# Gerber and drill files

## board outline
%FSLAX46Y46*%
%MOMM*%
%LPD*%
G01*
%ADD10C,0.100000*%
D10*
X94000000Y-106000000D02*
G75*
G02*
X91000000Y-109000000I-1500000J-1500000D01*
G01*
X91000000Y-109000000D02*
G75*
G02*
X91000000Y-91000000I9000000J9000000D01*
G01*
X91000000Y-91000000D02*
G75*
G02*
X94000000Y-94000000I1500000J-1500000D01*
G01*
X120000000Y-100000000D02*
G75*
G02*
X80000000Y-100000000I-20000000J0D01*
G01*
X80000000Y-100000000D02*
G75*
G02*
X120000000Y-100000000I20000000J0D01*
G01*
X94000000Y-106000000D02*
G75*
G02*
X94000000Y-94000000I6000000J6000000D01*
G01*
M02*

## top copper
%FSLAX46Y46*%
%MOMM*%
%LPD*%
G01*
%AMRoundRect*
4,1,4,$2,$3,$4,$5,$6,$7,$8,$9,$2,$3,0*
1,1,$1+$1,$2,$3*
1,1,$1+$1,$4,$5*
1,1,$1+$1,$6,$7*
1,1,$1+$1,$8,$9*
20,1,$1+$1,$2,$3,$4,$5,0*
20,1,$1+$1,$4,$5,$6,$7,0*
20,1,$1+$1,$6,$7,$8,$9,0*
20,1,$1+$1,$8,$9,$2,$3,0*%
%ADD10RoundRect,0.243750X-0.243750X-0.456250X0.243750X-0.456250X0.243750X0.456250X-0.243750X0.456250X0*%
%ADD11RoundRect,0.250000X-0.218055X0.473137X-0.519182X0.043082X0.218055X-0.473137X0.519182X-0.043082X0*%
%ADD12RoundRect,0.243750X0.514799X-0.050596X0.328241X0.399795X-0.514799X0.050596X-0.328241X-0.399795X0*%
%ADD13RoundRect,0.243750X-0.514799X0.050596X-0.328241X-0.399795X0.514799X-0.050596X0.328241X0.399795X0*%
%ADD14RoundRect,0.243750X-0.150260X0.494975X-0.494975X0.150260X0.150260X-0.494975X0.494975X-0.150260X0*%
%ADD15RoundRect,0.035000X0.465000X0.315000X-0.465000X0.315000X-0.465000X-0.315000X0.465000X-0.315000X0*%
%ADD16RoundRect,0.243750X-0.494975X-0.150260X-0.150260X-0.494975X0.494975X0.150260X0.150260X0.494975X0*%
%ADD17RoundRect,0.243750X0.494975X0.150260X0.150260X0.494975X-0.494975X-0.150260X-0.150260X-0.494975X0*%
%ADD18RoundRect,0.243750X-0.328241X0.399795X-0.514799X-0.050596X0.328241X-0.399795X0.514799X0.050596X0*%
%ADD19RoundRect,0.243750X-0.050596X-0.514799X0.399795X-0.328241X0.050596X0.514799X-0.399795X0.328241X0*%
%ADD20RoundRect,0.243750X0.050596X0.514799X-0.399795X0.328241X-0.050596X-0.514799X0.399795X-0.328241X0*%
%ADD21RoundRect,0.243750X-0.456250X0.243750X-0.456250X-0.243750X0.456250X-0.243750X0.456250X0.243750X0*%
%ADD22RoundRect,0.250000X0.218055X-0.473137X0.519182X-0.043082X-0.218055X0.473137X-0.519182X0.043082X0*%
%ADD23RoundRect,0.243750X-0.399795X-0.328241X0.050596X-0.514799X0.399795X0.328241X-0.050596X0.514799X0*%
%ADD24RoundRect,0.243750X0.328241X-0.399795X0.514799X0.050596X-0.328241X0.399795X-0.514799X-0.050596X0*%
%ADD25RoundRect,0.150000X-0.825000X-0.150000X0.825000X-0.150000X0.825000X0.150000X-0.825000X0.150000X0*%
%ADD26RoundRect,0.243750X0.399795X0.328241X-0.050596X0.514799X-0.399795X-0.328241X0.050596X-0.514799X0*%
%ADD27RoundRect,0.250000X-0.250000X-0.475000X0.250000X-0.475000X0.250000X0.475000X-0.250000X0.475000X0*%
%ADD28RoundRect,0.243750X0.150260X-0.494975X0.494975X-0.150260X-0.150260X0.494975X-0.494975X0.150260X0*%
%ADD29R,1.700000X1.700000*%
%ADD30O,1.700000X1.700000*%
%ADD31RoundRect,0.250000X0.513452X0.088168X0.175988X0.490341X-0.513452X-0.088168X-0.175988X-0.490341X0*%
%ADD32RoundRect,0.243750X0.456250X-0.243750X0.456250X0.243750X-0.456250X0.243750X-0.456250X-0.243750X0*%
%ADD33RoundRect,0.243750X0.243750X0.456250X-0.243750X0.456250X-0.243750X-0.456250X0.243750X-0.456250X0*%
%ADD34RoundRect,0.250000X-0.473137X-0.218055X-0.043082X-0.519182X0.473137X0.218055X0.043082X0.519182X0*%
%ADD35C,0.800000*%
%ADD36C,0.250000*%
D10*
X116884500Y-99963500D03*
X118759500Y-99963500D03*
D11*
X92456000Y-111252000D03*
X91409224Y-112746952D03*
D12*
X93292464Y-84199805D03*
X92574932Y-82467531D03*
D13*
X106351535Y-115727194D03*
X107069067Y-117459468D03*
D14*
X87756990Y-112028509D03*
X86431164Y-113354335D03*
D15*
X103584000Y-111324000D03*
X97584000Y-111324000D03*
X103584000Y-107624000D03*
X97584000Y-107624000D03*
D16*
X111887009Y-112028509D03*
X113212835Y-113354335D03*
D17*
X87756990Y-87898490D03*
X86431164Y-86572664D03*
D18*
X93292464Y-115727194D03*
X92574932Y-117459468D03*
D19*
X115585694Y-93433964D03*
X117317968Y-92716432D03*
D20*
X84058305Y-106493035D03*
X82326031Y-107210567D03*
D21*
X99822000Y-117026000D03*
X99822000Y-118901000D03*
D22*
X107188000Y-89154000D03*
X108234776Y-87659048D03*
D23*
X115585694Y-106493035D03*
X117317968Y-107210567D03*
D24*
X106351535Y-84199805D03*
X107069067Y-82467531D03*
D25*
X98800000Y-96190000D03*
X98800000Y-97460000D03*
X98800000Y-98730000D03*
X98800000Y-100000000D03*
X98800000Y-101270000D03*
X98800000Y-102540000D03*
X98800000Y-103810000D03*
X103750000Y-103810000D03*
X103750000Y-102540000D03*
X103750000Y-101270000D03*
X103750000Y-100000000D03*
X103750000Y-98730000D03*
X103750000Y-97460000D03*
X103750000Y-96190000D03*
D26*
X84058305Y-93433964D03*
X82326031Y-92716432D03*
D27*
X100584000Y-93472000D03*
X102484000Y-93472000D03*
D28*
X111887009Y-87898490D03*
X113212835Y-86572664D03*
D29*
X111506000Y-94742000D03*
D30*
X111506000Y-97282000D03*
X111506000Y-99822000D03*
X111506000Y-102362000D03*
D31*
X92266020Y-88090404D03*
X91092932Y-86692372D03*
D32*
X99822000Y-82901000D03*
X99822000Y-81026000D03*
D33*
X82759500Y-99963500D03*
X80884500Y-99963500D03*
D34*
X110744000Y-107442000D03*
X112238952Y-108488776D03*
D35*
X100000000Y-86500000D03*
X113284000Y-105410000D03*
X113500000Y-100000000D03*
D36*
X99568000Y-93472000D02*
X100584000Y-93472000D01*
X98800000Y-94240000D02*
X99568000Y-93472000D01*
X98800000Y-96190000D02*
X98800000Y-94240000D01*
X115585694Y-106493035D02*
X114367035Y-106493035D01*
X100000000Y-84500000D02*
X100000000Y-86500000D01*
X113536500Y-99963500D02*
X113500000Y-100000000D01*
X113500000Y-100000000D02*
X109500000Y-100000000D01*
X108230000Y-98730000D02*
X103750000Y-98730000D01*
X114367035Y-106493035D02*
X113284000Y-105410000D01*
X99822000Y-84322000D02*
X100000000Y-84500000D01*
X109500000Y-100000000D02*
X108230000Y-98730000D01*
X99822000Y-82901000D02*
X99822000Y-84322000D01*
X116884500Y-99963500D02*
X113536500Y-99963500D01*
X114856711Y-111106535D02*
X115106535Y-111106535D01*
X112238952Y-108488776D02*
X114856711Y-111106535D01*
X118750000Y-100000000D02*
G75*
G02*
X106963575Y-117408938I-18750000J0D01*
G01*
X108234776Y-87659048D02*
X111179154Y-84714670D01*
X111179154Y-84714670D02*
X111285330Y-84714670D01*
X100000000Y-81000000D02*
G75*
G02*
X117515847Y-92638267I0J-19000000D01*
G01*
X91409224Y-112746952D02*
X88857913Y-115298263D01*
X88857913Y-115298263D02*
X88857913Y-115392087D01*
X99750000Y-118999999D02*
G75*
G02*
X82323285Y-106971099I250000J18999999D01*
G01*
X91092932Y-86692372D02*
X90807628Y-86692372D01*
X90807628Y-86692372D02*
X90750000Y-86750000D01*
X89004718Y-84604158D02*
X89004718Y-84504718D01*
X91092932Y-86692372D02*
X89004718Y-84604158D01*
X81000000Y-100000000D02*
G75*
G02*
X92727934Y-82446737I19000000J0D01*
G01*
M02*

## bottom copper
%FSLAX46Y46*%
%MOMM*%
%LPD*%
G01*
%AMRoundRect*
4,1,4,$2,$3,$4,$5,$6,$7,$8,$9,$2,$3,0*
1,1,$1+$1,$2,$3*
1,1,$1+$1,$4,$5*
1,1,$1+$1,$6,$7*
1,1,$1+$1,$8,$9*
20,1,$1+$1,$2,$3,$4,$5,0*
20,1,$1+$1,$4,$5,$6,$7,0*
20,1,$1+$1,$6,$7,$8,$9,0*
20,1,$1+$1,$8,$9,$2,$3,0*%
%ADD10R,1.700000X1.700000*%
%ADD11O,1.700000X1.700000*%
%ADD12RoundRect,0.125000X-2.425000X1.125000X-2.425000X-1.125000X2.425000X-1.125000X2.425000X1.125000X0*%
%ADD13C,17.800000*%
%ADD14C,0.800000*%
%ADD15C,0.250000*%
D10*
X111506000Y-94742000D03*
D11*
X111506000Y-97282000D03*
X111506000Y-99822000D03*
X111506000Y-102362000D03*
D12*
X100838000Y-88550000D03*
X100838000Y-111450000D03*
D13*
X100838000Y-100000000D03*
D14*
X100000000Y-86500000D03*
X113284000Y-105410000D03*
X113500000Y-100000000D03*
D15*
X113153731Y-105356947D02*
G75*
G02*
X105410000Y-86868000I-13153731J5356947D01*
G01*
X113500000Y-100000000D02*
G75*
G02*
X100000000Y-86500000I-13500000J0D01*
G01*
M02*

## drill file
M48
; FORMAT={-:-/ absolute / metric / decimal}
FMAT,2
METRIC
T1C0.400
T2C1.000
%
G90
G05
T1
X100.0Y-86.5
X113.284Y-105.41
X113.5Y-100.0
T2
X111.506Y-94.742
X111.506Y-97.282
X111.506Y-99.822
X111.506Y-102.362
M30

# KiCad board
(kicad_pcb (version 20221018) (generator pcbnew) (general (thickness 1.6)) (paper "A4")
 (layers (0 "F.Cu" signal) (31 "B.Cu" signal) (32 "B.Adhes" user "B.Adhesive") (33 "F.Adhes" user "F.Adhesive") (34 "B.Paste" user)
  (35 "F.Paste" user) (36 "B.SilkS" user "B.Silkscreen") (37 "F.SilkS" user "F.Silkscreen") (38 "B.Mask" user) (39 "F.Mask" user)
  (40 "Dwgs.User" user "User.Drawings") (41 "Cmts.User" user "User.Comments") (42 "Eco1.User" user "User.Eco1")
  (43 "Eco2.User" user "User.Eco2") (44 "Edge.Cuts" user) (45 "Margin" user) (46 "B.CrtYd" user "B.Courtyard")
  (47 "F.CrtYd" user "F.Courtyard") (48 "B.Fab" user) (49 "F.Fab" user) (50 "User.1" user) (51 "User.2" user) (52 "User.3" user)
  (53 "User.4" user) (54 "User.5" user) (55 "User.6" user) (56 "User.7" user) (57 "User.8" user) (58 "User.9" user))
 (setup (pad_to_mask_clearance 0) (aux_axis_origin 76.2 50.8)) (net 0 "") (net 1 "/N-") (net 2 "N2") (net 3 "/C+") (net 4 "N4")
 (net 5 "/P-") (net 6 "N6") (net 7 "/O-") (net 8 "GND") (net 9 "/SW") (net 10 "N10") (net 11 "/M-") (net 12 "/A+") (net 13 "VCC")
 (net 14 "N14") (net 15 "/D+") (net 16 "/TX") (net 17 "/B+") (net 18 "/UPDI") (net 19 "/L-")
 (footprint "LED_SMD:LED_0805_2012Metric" (layer "F.Cu") (at 117.822 99.9635)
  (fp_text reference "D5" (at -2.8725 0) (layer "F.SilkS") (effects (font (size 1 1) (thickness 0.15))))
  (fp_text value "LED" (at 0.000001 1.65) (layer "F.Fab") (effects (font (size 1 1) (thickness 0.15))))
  (pad "1" smd roundrect (at -0.9375 0) (size 0.975 1.4) (layers "F.Cu" "F.Paste" "F.Mask") (roundrect_rratio 0.25) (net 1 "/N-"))
  (pad "2" smd roundrect (at 0.9375 0) (size 0.975 1.4) (layers "F.Cu" "F.Paste" "F.Mask") (roundrect_rratio 0.25) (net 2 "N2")))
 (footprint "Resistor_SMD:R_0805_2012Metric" (layer "F.Cu") (at 91.932612 111.999476 -125)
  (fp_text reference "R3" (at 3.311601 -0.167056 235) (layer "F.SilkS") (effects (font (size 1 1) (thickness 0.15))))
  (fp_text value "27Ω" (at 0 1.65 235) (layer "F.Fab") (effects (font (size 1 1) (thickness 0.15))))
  (pad "1" smd roundrect (at -0.9125 0 235) (size 1.025 1.4) (layers "F.Cu" "F.Paste" "F.Mask") (roundrect_rratio 0.243902) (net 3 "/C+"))
  (pad "2" smd roundrect (at 0.9125 0 235) (size 1.025 1.4) (layers "F.Cu" "F.Paste" "F.Mask") (roundrect_rratio 0.243902) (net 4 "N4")))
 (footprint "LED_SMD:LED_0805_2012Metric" (layer "F.Cu") (at 92.933698 83.333668 112.5)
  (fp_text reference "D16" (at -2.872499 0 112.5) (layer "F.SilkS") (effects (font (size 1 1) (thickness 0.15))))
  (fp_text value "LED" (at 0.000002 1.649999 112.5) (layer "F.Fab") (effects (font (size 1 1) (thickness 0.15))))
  (pad "1" smd roundrect (at -0.9375 0 112.5) (size 0.975 1.4) (layers "F.Cu" "F.Paste" "F.Mask") (roundrect_rratio 0.25) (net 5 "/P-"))
  (pad "2" smd roundrect (at 0.9375 0 112.5) (size 0.975 1.4) (layers "F.Cu" "F.Paste" "F.Mask") (roundrect_rratio 0.25) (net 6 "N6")))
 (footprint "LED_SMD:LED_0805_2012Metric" (layer "F.Cu") (at 106.710301 116.593331 -67.5)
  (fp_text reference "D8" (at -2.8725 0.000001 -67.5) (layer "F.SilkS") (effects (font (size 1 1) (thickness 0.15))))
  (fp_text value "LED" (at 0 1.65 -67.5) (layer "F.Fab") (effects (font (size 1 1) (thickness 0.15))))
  (pad "1" smd roundrect (at -0.9375 0 292.5) (size 0.975 1.4) (layers "F.Cu" "F.Paste" "F.Mask") (roundrect_rratio 0.25) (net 5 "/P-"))
  (pad "2" smd roundrect (at 0.9375 0 292.5) (size 0.975 1.4) (layers "F.Cu" "F.Paste" "F.Mask") (roundrect_rratio 0.25) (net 2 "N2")))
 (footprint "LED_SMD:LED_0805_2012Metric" (layer "F.Cu") (at 87.094077 112.691422 -135)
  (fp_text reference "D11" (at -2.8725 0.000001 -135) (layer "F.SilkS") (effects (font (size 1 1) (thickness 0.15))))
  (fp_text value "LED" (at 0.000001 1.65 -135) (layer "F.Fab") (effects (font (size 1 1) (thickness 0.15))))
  (pad "1" smd roundrect (at -0.9375 0 225) (size 0.975 1.4) (layers "F.Cu" "F.Paste" "F.Mask") (roundrect_rratio 0.25) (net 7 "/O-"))
  (pad "2" smd roundrect (at 0.9375 0 225) (size 0.975 1.4) (layers "F.Cu" "F.Paste" "F.Mask") (roundrect_rratio 0.25) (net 4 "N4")))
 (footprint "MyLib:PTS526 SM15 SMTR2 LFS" (layer "F.Cu") (at 100.584 109.474 180)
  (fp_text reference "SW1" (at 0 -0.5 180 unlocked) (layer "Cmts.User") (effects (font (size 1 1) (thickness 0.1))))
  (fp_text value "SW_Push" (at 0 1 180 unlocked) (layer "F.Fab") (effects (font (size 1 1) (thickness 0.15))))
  (pad "1" smd roundrect (at -3 -1.85 180) (size 1 0.7) (layers "F.Cu" "F.Paste" "F.Mask") (roundrect_rratio 0.05) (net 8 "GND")
   (thermal_bridge_angle 45))
  (pad "1" smd roundrect (at 3 -1.85 180) (size 1 0.7) (layers "F.Cu" "F.Paste" "F.Mask") (roundrect_rratio 0.05) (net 8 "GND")
   (thermal_bridge_angle 45))
  (pad "2" smd roundrect (at -3 1.85 180) (size 1 0.7) (layers "F.Cu" "F.Paste" "F.Mask") (roundrect_rratio 0.05) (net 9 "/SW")
   (thermal_bridge_angle 45))
  (pad "2" smd roundrect (at 3 1.85 180) (size 1 0.7) (layers "F.Cu" "F.Paste" "F.Mask") (roundrect_rratio 0.05) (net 9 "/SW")
   (thermal_bridge_angle 45)))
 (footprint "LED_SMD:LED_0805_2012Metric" (layer "F.Cu") (at 112.549922 112.691422 -45)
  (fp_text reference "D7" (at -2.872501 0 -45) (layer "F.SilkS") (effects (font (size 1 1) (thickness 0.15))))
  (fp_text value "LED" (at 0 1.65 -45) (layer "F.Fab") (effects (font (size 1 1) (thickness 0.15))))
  (pad "1" smd roundrect (at -0.9375 0 315) (size 0.975 1.4) (layers "F.Cu" "F.Paste" "F.Mask") (roundrect_rratio 0.25) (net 7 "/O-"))
  (pad "2" smd roundrect (at 0.9375 0 315) (size 0.975 1.4) (layers "F.Cu" "F.Paste" "F.Mask") (roundrect_rratio 0.25) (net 2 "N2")))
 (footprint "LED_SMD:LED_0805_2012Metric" (layer "F.Cu") (at 87.094077 87.235577 135)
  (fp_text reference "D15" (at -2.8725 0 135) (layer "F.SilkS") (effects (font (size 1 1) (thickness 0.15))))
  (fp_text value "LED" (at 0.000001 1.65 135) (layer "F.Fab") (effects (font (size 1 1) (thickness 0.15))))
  (pad "1" smd roundrect (at -0.9375 0 135) (size 0.975 1.4) (layers "F.Cu" "F.Paste" "F.Mask") (roundrect_rratio 0.25) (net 7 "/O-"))
  (pad "2" smd roundrect (at 0.9375 0 135) (size 0.975 1.4) (layers "F.Cu" "F.Paste" "F.Mask") (roundrect_rratio 0.25) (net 6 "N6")))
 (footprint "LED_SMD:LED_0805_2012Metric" (layer "F.Cu") (at 92.933698 116.593331 -112.5)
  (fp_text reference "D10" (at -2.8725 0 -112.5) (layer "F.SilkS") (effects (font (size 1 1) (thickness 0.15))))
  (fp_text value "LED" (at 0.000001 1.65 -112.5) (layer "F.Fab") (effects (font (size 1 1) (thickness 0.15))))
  (pad "1" smd roundrect (at -0.9375 0 247.5) (size 0.975 1.4) (layers "F.Cu" "F.Paste" "F.Mask") (roundrect_rratio 0.25) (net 1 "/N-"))
  (pad "2" smd roundrect (at 0.9375 0 247.5) (size 0.975 1.4) (layers "F.Cu" "F.Paste" "F.Mask") (roundrect_rratio 0.25) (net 4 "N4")))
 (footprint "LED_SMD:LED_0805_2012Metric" (layer "F.Cu") (at 116.451831 93.075198 22.5)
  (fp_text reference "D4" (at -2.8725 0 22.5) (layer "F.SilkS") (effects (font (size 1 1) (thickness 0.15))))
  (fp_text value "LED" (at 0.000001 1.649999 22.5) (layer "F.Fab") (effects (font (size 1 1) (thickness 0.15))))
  (pad "1" smd roundrect (at -0.9375 0 22.5) (size 0.975 1.4) (layers "F.Cu" "F.Paste" "F.Mask") (roundrect_rratio 0.25) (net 5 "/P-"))
  (pad "2" smd roundrect (at 0.9375 0 22.5) (size 0.975 1.4) (layers "F.Cu" "F.Paste" "F.Mask") (roundrect_rratio 0.25) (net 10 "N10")))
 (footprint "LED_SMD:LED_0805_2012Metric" (layer "F.Cu") (at 83.192168 106.851801 -157.5)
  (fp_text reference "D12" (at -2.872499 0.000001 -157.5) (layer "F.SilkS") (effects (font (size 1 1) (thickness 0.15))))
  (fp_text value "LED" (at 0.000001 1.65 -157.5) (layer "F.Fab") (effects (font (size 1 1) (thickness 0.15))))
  (pad "1" smd roundrect (at -0.9375 0 202.5) (size 0.975 1.4) (layers "F.Cu" "F.Paste" "F.Mask") (roundrect_rratio 0.25) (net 5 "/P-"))
  (pad "2" smd roundrect (at 0.9375 0 202.5) (size 0.975 1.4) (layers "F.Cu" "F.Paste" "F.Mask") (roundrect_rratio 0.25) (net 4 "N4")))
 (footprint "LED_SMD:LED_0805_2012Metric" (layer "F.Cu") (at 99.822 117.9635 -90)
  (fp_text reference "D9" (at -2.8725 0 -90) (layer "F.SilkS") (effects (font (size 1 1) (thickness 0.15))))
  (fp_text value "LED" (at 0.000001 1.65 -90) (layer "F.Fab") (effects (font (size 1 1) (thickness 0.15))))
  (pad "1" smd roundrect (at -0.9375 0 270) (size 0.975 1.4) (layers "F.Cu" "F.Paste" "F.Mask") (roundrect_rratio 0.25) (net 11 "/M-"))
  (pad "2" smd roundrect (at 0.9375 0 270) (size 0.975 1.4) (layers "F.Cu" "F.Paste" "F.Mask") (roundrect_rratio 0.25) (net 4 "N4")))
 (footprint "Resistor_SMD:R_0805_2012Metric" (layer "F.Cu") (at 107.711388 88.406524 55)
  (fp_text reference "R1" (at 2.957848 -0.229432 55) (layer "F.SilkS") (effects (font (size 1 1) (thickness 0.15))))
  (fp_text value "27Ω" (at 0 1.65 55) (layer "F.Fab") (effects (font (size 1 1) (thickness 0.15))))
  (pad "1" smd roundrect (at -0.9125 0 55) (size 1.025 1.4) (layers "F.Cu" "F.Paste" "F.Mask") (roundrect_rratio 0.243902) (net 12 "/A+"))
  (pad "2" smd roundrect (at 0.9125 0 55) (size 1.025 1.4) (layers "F.Cu" "F.Paste" "F.Mask") (roundrect_rratio 0.243902) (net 10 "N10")))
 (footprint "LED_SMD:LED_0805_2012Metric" (layer "F.Cu") (at 116.451831 106.851801 -22.5)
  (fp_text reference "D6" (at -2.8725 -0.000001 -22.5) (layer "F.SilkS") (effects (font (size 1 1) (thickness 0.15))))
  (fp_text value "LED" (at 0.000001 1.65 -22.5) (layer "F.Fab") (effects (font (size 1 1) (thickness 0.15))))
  (pad "1" smd roundrect (at -0.9375 0 337.5) (size 0.975 1.4) (layers "F.Cu" "F.Paste" "F.Mask") (roundrect_rratio 0.25) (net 1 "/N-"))
  (pad "2" smd roundrect (at 0.9375 0 337.5) (size 0.975 1.4) (layers "F.Cu" "F.Paste" "F.Mask") (roundrect_rratio 0.25) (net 2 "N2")))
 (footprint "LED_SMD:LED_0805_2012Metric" (layer "F.Cu") (at 106.710301 83.333668 67.5)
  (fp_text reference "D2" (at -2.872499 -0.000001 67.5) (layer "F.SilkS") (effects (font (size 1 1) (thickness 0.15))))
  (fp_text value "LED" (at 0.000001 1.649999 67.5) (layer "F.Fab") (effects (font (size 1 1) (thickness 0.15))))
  (pad "1" smd roundrect (at -0.9375 0 67.5) (size 0.975 1.4) (layers "F.Cu" "F.Paste" "F.Mask") (roundrect_rratio 0.25) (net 1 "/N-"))
  (pad "2" smd roundrect (at 0.9375 0 67.5) (size 0.975 1.4) (layers "F.Cu" "F.Paste" "F.Mask") (roundrect_rratio 0.25) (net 10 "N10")))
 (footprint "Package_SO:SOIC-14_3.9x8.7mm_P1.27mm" (layer "F.Cu") (at 101.275 100)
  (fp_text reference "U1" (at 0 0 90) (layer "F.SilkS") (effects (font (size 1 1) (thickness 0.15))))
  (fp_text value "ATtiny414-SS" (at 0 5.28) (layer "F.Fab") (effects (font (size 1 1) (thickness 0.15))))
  (pad "1" smd roundrect (at -2.475 -3.81) (size 1.95 0.6) (layers "F.Cu" "F.Paste" "F.Mask") (roundrect_rratio 0.25) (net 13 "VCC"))
  (pad "2" smd roundrect (at -2.475 -2.54) (size 1.95 0.6) (layers "F.Cu" "F.Paste" "F.Mask") (roundrect_rratio 0.25) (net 7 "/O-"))
  (pad "3" smd roundrect (at -2.475 -1.27) (size 1.95 0.6) (layers "F.Cu" "F.Paste" "F.Mask") (roundrect_rratio 0.25) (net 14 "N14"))
  (pad "4" smd roundrect (at -2.475 0) (size 1.95 0.6) (layers "F.Cu" "F.Paste" "F.Mask") (roundrect_rratio 0.25) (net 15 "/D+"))
  (pad "5" smd roundrect (at -2.475 1.27) (size 1.95 0.6) (layers "F.Cu" "F.Paste" "F.Mask") (roundrect_rratio 0.25) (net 9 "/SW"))
  (pad "6" smd roundrect (at -2.475 2.54) (size 1.95 0.6) (layers "F.Cu" "F.Paste" "F.Mask") (roundrect_rratio 0.25) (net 3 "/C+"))
  (pad "7" smd roundrect (at -2.475 3.81) (size 1.95 0.6) (layers "F.Cu" "F.Paste" "F.Mask") (roundrect_rratio 0.25) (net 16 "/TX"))
  (pad "8" smd roundrect (at 2.475 3.81) (size 1.95 0.6) (layers "F.Cu" "F.Paste" "F.Mask") (roundrect_rratio 0.25) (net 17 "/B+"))
  (pad "9" smd roundrect (at 2.475 2.54) (size 1.95 0.6) (layers "F.Cu" "F.Paste" "F.Mask") (roundrect_rratio 0.25) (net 12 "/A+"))
  (pad "10" smd roundrect (at 2.475 1.27) (size 1.95 0.6) (layers "F.Cu" "F.Paste" "F.Mask") (roundrect_rratio 0.25) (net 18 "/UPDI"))
  (pad "11" smd roundrect (at 2.475 0) (size 1.95 0.6) (layers "F.Cu" "F.Paste" "F.Mask") (roundrect_rratio 0.25) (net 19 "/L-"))
  (pad "12" smd roundrect (at 2.475 -1.27) (size 1.95 0.6) (layers "F.Cu" "F.Paste" "F.Mask") (roundrect_rratio 0.25) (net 1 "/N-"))
  (pad "13" smd roundrect (at 2.475 -2.54) (size 1.95 0.6) (layers "F.Cu" "F.Paste" "F.Mask") (roundrect_rratio 0.25) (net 1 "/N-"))
  (pad "14" smd roundrect (at 2.475 -3.81) (size 1.95 0.6) (layers "F.Cu" "F.Paste" "F.Mask") (roundrect_rratio 0.25) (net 8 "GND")))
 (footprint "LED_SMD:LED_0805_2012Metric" (layer "F.Cu") (at 83.192168 93.075198 157.5)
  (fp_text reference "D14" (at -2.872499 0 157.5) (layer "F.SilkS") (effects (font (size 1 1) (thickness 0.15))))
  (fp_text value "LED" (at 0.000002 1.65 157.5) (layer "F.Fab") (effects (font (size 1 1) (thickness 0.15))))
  (pad "1" smd roundrect (at -0.9375 0 157.5) (size 0.975 1.4) (layers "F.Cu" "F.Paste" "F.Mask") (roundrect_rratio 0.25) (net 1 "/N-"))
  (pad "2" smd roundrect (at 0.9375 0 157.5) (size 0.975 1.4) (layers "F.Cu" "F.Paste" "F.Mask") (roundrect_rratio 0.25) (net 6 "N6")))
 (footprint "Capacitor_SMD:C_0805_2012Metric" (layer "F.Cu") (at 101.534 93.472)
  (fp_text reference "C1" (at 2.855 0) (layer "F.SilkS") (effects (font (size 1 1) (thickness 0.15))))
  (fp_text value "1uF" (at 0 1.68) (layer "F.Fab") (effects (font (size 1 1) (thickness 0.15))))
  (pad "1" smd roundrect (at -0.95 0) (size 1 1.45) (layers "F.Cu" "F.Paste" "F.Mask") (roundrect_rratio 0.25) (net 13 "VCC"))
  (pad "2" smd roundrect (at 0.95 0) (size 1 1.45) (layers "F.Cu" "F.Paste" "F.Mask") (roundrect_rratio 0.25) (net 8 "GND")))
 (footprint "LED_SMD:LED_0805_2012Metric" (layer "F.Cu") (at 112.549922 87.235577 45)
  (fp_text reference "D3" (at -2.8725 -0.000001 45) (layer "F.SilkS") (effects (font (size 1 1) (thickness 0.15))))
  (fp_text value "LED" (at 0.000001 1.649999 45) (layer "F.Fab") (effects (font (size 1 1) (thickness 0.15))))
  (pad "1" smd roundrect (at -0.9375 0 45) (size 0.975 1.4) (layers "F.Cu" "F.Paste" "F.Mask") (roundrect_rratio 0.25) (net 7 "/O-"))
  (pad "2" smd roundrect (at 0.9375 0 45) (size 0.975 1.4) (layers "F.Cu" "F.Paste" "F.Mask") (roundrect_rratio 0.25) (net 10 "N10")))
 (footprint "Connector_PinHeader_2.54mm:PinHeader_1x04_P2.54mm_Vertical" (layer "F.Cu") (at 111.506 94.742)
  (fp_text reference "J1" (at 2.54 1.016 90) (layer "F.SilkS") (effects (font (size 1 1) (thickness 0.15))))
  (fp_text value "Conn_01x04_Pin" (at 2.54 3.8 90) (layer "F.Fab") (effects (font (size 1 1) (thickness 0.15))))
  (pad "1" thru_hole rect (at 0 0) (size 1.7 1.7) (drill 1) (layers "*.Cu" "*.Mask") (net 8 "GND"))
  (pad "2" thru_hole oval (at 0 2.54) (size 1.7 1.7) (drill 1) (layers "*.Cu" "*.Mask") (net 13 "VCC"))
  (pad "3" thru_hole oval (at 0 5.08) (size 1.7 1.7) (drill 1) (layers "*.Cu" "*.Mask") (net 16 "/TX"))
  (pad "4" thru_hole oval (at 0 7.62) (size 1.7 1.7) (drill 1) (layers "*.Cu" "*.Mask") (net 18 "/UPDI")))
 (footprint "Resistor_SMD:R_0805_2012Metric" (layer "F.Cu") (at 91.679476 87.391388 130)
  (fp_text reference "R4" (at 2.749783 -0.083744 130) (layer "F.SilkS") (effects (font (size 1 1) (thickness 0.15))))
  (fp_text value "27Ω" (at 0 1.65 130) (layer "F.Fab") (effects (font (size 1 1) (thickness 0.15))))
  (pad "1" smd roundrect (at -0.9125 0 130) (size 1.025 1.4) (layers "F.Cu" "F.Paste" "F.Mask") (roundrect_rratio 0.243902) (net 15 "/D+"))
  (pad "2" smd roundrect (at 0.9125 0 130) (size 1.025 1.4) (layers "F.Cu" "F.Paste" "F.Mask") (roundrect_rratio 0.243902) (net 6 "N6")))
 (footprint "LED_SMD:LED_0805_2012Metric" (layer "F.Cu") (at 99.822 81.9635 90)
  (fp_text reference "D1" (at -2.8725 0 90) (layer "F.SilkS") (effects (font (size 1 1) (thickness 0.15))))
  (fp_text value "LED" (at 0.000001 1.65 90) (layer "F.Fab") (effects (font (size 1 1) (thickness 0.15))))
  (pad "1" smd roundrect (at -0.9375 0 90) (size 0.975 1.4) (layers "F.Cu" "F.Paste" "F.Mask") (roundrect_rratio 0.25) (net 1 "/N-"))
  (pad "2" smd roundrect (at 0.9375 0 90) (size 0.975 1.4) (layers "F.Cu" "F.Paste" "F.Mask") (roundrect_rratio 0.25) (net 10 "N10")))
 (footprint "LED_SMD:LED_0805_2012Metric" (layer "F.Cu") (at 81.822 99.9635 180)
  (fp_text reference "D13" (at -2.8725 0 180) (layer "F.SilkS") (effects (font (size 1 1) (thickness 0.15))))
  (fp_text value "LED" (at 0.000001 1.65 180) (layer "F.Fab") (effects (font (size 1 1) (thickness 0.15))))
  (pad "1" smd roundrect (at -0.9375 0 180) (size 0.975 1.4) (layers "F.Cu" "F.Paste" "F.Mask") (roundrect_rratio 0.25) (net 11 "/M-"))
  (pad "2" smd roundrect (at 0.9375 0 180) (size 0.975 1.4) (layers "F.Cu" "F.Paste" "F.Mask") (roundrect_rratio 0.25) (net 6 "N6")))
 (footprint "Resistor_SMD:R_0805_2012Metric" (layer "F.Cu") (at 111.491476 107.965388 -35)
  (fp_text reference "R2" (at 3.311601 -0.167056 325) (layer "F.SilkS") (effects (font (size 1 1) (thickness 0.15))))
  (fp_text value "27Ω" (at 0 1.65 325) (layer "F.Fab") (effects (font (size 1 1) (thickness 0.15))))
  (pad "1" smd roundrect (at -0.9125 0 325) (size 1.025 1.4) (layers "F.Cu" "F.Paste" "F.Mask") (roundrect_rratio 0.243902) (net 17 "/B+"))
  (pad "2" smd roundrect (at 0.9125 0 325) (size 1.025 1.4) (layers "F.Cu" "F.Paste" "F.Mask") (roundrect_rratio 0.243902) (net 2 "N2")))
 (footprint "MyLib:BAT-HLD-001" (layer "B.Cu") (at 100.838 100 -90)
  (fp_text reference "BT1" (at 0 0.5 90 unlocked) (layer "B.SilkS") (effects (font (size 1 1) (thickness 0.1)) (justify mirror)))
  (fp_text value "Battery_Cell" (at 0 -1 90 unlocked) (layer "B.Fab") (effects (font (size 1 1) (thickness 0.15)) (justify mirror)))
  (pad "1" smd roundrect (at -11.45 0 270) (size 2.5 5.1) (layers "B.Cu" "B.Paste" "B.Mask") (roundrect_rratio 0.05) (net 11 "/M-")
   (thermal_bridge_angle 45))
  (pad "1" smd roundrect (at 11.45 0 270) (size 2.5 5.1) (layers "B.Cu" "B.Paste" "B.Mask") (roundrect_rratio 0.05) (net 1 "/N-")
   (thermal_bridge_angle 45))
  (pad "2" smd circle (at 0 0 270) (size 17.8 17.8) (layers "B.Cu" "B.Paste" "B.Mask") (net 1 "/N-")))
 (gr_arc (start 94 106) (mid 94 109) (end 91 109) (stroke (width 0.1) (type default)) (layer "Edge.Cuts"))
 (gr_arc (start 91 109) (mid 87.272078 100) (end 91 91) (stroke (width 0.1) (type default)) (layer "Edge.Cuts"))
 (gr_arc (start 91 91) (mid 94 91) (end 94 94) (stroke (width 0.1) (type default)) (layer "Edge.Cuts"))
 (gr_circle (center 100 100) (end 120 100) (stroke (width 0.1) (type default)) (fill none) (layer "Edge.Cuts"))
 (gr_arc (start 94 106) (mid 91.514719 100) (end 94 94) (stroke (width 0.1) (type default)) (layer "Edge.Cuts"))
 (segment (start 99.568 93.472) (end 100.584 93.472) (width 0.25) (layer "F.Cu") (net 13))
 (segment (start 98.8 94.24) (end 99.568 93.472) (width 0.25) (layer "F.Cu") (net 13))
 (segment (start 98.8 96.19) (end 98.8 94.24) (width 0.25) (layer "F.Cu") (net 13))
 (segment (start 115.585694 106.493035) (end 114.367035 106.493035) (width 0.25) (layer "F.Cu") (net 1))
 (segment (start 100 84.5) (end 100 86.5) (width 0.25) (layer "F.Cu") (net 1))
 (segment (start 113.5365 99.9635) (end 113.5 100) (width 0.25) (layer "F.Cu") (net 1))
 (segment (start 113.5 100) (end 109.5 100) (width 0.25) (layer "F.Cu") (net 1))
 (segment (start 108.23 98.73) (end 103.75 98.73) (width 0.25) (layer "F.Cu") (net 1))
 (segment (start 114.367035 106.493035) (end 113.284 105.41) (width 0.25) (layer "F.Cu") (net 1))
 (segment (start 99.822 84.322) (end 100 84.5) (width 0.25) (layer "F.Cu") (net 1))
 (segment (start 109.5 100) (end 108.23 98.73) (width 0.25) (layer "F.Cu") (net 1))
 (segment (start 99.822 82.901) (end 99.822 84.322) (width 0.25) (layer "F.Cu") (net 1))
 (segment (start 116.8845 99.9635) (end 113.5365 99.9635) (width 0.25) (layer "F.Cu") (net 1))
 (via (at 100 86.5) (size 0.8) (drill 0.4) (layers "F.Cu" "B.Cu") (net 1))
 (via (at 113.284 105.41) (size 0.8) (drill 0.4) (layers "F.Cu" "B.Cu") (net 1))
 (via (at 113.5 100) (size 0.8) (drill 0.4) (layers "F.Cu" "B.Cu") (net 1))
 (arc (start 113.153731 105.356947) (mid 86.899873 105.48673) (end 105.41 86.868) (width 0.25) (layer "B.Cu") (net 1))
 (arc (start 113.5 100) (mid 90.454058 109.545942) (end 100 86.5) (width 0.25) (layer "B.Cu") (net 1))
 (segment (start 114.856711 111.106535) (end 115.106535 111.106535) (width 0.25) (layer "F.Cu") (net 2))
 (segment (start 112.238952 108.488776) (end 114.856711 111.106535) (width 0.25) (layer "F.Cu") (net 2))
 (arc (start 118.75 100) (mid 115.526261 110.51179) (end 106.963575 117.408938) (width 0.25) (layer "F.Cu") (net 2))
 (segment (start 108.234776 87.659048) (end 111.179154 84.71467) (width 0.25) (layer "F.Cu") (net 10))
 (segment (start 111.179154 84.71467) (end 111.28533 84.71467) (width 0.25) (layer "F.Cu") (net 10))
 (arc (start 100 81) (mid 110.51492 84.174816) (end 117.515847 92.638267) (width 0.25) (layer "F.Cu") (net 10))
 (segment (start 91.409224 112.746952) (end 88.857913 115.298263) (width 0.25) (layer "F.Cu") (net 4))
 (segment (start 88.857913 115.298263) (end 88.857913 115.392087) (width 0.25) (layer "F.Cu") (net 4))
 (arc (start 99.75 118.999999) (mid 89.205771 115.638001) (end 82.323285 106.971099) (width 0.25) (layer "F.Cu") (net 4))
 (segment (start 91.092932 86.692372) (end 90.807628 86.692372) (width 0.25) (layer "F.Cu") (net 6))
 (segment (start 90.807628 86.692372) (end 90.75 86.75) (width 0.25) (layer "F.Cu") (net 6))
 (segment (start 89.004718 84.604158) (end 89.004718 84.504718) (width 0.25) (layer "F.Cu") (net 6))
 (segment (start 91.092932 86.692372) (end 89.004718 84.604158) (width 0.25) (layer "F.Cu") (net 6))
 (arc (start 81 100) (mid 84.201752 89.444652) (end 92.727934 82.446737) (width 0.25) (layer "F.Cu") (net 6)))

